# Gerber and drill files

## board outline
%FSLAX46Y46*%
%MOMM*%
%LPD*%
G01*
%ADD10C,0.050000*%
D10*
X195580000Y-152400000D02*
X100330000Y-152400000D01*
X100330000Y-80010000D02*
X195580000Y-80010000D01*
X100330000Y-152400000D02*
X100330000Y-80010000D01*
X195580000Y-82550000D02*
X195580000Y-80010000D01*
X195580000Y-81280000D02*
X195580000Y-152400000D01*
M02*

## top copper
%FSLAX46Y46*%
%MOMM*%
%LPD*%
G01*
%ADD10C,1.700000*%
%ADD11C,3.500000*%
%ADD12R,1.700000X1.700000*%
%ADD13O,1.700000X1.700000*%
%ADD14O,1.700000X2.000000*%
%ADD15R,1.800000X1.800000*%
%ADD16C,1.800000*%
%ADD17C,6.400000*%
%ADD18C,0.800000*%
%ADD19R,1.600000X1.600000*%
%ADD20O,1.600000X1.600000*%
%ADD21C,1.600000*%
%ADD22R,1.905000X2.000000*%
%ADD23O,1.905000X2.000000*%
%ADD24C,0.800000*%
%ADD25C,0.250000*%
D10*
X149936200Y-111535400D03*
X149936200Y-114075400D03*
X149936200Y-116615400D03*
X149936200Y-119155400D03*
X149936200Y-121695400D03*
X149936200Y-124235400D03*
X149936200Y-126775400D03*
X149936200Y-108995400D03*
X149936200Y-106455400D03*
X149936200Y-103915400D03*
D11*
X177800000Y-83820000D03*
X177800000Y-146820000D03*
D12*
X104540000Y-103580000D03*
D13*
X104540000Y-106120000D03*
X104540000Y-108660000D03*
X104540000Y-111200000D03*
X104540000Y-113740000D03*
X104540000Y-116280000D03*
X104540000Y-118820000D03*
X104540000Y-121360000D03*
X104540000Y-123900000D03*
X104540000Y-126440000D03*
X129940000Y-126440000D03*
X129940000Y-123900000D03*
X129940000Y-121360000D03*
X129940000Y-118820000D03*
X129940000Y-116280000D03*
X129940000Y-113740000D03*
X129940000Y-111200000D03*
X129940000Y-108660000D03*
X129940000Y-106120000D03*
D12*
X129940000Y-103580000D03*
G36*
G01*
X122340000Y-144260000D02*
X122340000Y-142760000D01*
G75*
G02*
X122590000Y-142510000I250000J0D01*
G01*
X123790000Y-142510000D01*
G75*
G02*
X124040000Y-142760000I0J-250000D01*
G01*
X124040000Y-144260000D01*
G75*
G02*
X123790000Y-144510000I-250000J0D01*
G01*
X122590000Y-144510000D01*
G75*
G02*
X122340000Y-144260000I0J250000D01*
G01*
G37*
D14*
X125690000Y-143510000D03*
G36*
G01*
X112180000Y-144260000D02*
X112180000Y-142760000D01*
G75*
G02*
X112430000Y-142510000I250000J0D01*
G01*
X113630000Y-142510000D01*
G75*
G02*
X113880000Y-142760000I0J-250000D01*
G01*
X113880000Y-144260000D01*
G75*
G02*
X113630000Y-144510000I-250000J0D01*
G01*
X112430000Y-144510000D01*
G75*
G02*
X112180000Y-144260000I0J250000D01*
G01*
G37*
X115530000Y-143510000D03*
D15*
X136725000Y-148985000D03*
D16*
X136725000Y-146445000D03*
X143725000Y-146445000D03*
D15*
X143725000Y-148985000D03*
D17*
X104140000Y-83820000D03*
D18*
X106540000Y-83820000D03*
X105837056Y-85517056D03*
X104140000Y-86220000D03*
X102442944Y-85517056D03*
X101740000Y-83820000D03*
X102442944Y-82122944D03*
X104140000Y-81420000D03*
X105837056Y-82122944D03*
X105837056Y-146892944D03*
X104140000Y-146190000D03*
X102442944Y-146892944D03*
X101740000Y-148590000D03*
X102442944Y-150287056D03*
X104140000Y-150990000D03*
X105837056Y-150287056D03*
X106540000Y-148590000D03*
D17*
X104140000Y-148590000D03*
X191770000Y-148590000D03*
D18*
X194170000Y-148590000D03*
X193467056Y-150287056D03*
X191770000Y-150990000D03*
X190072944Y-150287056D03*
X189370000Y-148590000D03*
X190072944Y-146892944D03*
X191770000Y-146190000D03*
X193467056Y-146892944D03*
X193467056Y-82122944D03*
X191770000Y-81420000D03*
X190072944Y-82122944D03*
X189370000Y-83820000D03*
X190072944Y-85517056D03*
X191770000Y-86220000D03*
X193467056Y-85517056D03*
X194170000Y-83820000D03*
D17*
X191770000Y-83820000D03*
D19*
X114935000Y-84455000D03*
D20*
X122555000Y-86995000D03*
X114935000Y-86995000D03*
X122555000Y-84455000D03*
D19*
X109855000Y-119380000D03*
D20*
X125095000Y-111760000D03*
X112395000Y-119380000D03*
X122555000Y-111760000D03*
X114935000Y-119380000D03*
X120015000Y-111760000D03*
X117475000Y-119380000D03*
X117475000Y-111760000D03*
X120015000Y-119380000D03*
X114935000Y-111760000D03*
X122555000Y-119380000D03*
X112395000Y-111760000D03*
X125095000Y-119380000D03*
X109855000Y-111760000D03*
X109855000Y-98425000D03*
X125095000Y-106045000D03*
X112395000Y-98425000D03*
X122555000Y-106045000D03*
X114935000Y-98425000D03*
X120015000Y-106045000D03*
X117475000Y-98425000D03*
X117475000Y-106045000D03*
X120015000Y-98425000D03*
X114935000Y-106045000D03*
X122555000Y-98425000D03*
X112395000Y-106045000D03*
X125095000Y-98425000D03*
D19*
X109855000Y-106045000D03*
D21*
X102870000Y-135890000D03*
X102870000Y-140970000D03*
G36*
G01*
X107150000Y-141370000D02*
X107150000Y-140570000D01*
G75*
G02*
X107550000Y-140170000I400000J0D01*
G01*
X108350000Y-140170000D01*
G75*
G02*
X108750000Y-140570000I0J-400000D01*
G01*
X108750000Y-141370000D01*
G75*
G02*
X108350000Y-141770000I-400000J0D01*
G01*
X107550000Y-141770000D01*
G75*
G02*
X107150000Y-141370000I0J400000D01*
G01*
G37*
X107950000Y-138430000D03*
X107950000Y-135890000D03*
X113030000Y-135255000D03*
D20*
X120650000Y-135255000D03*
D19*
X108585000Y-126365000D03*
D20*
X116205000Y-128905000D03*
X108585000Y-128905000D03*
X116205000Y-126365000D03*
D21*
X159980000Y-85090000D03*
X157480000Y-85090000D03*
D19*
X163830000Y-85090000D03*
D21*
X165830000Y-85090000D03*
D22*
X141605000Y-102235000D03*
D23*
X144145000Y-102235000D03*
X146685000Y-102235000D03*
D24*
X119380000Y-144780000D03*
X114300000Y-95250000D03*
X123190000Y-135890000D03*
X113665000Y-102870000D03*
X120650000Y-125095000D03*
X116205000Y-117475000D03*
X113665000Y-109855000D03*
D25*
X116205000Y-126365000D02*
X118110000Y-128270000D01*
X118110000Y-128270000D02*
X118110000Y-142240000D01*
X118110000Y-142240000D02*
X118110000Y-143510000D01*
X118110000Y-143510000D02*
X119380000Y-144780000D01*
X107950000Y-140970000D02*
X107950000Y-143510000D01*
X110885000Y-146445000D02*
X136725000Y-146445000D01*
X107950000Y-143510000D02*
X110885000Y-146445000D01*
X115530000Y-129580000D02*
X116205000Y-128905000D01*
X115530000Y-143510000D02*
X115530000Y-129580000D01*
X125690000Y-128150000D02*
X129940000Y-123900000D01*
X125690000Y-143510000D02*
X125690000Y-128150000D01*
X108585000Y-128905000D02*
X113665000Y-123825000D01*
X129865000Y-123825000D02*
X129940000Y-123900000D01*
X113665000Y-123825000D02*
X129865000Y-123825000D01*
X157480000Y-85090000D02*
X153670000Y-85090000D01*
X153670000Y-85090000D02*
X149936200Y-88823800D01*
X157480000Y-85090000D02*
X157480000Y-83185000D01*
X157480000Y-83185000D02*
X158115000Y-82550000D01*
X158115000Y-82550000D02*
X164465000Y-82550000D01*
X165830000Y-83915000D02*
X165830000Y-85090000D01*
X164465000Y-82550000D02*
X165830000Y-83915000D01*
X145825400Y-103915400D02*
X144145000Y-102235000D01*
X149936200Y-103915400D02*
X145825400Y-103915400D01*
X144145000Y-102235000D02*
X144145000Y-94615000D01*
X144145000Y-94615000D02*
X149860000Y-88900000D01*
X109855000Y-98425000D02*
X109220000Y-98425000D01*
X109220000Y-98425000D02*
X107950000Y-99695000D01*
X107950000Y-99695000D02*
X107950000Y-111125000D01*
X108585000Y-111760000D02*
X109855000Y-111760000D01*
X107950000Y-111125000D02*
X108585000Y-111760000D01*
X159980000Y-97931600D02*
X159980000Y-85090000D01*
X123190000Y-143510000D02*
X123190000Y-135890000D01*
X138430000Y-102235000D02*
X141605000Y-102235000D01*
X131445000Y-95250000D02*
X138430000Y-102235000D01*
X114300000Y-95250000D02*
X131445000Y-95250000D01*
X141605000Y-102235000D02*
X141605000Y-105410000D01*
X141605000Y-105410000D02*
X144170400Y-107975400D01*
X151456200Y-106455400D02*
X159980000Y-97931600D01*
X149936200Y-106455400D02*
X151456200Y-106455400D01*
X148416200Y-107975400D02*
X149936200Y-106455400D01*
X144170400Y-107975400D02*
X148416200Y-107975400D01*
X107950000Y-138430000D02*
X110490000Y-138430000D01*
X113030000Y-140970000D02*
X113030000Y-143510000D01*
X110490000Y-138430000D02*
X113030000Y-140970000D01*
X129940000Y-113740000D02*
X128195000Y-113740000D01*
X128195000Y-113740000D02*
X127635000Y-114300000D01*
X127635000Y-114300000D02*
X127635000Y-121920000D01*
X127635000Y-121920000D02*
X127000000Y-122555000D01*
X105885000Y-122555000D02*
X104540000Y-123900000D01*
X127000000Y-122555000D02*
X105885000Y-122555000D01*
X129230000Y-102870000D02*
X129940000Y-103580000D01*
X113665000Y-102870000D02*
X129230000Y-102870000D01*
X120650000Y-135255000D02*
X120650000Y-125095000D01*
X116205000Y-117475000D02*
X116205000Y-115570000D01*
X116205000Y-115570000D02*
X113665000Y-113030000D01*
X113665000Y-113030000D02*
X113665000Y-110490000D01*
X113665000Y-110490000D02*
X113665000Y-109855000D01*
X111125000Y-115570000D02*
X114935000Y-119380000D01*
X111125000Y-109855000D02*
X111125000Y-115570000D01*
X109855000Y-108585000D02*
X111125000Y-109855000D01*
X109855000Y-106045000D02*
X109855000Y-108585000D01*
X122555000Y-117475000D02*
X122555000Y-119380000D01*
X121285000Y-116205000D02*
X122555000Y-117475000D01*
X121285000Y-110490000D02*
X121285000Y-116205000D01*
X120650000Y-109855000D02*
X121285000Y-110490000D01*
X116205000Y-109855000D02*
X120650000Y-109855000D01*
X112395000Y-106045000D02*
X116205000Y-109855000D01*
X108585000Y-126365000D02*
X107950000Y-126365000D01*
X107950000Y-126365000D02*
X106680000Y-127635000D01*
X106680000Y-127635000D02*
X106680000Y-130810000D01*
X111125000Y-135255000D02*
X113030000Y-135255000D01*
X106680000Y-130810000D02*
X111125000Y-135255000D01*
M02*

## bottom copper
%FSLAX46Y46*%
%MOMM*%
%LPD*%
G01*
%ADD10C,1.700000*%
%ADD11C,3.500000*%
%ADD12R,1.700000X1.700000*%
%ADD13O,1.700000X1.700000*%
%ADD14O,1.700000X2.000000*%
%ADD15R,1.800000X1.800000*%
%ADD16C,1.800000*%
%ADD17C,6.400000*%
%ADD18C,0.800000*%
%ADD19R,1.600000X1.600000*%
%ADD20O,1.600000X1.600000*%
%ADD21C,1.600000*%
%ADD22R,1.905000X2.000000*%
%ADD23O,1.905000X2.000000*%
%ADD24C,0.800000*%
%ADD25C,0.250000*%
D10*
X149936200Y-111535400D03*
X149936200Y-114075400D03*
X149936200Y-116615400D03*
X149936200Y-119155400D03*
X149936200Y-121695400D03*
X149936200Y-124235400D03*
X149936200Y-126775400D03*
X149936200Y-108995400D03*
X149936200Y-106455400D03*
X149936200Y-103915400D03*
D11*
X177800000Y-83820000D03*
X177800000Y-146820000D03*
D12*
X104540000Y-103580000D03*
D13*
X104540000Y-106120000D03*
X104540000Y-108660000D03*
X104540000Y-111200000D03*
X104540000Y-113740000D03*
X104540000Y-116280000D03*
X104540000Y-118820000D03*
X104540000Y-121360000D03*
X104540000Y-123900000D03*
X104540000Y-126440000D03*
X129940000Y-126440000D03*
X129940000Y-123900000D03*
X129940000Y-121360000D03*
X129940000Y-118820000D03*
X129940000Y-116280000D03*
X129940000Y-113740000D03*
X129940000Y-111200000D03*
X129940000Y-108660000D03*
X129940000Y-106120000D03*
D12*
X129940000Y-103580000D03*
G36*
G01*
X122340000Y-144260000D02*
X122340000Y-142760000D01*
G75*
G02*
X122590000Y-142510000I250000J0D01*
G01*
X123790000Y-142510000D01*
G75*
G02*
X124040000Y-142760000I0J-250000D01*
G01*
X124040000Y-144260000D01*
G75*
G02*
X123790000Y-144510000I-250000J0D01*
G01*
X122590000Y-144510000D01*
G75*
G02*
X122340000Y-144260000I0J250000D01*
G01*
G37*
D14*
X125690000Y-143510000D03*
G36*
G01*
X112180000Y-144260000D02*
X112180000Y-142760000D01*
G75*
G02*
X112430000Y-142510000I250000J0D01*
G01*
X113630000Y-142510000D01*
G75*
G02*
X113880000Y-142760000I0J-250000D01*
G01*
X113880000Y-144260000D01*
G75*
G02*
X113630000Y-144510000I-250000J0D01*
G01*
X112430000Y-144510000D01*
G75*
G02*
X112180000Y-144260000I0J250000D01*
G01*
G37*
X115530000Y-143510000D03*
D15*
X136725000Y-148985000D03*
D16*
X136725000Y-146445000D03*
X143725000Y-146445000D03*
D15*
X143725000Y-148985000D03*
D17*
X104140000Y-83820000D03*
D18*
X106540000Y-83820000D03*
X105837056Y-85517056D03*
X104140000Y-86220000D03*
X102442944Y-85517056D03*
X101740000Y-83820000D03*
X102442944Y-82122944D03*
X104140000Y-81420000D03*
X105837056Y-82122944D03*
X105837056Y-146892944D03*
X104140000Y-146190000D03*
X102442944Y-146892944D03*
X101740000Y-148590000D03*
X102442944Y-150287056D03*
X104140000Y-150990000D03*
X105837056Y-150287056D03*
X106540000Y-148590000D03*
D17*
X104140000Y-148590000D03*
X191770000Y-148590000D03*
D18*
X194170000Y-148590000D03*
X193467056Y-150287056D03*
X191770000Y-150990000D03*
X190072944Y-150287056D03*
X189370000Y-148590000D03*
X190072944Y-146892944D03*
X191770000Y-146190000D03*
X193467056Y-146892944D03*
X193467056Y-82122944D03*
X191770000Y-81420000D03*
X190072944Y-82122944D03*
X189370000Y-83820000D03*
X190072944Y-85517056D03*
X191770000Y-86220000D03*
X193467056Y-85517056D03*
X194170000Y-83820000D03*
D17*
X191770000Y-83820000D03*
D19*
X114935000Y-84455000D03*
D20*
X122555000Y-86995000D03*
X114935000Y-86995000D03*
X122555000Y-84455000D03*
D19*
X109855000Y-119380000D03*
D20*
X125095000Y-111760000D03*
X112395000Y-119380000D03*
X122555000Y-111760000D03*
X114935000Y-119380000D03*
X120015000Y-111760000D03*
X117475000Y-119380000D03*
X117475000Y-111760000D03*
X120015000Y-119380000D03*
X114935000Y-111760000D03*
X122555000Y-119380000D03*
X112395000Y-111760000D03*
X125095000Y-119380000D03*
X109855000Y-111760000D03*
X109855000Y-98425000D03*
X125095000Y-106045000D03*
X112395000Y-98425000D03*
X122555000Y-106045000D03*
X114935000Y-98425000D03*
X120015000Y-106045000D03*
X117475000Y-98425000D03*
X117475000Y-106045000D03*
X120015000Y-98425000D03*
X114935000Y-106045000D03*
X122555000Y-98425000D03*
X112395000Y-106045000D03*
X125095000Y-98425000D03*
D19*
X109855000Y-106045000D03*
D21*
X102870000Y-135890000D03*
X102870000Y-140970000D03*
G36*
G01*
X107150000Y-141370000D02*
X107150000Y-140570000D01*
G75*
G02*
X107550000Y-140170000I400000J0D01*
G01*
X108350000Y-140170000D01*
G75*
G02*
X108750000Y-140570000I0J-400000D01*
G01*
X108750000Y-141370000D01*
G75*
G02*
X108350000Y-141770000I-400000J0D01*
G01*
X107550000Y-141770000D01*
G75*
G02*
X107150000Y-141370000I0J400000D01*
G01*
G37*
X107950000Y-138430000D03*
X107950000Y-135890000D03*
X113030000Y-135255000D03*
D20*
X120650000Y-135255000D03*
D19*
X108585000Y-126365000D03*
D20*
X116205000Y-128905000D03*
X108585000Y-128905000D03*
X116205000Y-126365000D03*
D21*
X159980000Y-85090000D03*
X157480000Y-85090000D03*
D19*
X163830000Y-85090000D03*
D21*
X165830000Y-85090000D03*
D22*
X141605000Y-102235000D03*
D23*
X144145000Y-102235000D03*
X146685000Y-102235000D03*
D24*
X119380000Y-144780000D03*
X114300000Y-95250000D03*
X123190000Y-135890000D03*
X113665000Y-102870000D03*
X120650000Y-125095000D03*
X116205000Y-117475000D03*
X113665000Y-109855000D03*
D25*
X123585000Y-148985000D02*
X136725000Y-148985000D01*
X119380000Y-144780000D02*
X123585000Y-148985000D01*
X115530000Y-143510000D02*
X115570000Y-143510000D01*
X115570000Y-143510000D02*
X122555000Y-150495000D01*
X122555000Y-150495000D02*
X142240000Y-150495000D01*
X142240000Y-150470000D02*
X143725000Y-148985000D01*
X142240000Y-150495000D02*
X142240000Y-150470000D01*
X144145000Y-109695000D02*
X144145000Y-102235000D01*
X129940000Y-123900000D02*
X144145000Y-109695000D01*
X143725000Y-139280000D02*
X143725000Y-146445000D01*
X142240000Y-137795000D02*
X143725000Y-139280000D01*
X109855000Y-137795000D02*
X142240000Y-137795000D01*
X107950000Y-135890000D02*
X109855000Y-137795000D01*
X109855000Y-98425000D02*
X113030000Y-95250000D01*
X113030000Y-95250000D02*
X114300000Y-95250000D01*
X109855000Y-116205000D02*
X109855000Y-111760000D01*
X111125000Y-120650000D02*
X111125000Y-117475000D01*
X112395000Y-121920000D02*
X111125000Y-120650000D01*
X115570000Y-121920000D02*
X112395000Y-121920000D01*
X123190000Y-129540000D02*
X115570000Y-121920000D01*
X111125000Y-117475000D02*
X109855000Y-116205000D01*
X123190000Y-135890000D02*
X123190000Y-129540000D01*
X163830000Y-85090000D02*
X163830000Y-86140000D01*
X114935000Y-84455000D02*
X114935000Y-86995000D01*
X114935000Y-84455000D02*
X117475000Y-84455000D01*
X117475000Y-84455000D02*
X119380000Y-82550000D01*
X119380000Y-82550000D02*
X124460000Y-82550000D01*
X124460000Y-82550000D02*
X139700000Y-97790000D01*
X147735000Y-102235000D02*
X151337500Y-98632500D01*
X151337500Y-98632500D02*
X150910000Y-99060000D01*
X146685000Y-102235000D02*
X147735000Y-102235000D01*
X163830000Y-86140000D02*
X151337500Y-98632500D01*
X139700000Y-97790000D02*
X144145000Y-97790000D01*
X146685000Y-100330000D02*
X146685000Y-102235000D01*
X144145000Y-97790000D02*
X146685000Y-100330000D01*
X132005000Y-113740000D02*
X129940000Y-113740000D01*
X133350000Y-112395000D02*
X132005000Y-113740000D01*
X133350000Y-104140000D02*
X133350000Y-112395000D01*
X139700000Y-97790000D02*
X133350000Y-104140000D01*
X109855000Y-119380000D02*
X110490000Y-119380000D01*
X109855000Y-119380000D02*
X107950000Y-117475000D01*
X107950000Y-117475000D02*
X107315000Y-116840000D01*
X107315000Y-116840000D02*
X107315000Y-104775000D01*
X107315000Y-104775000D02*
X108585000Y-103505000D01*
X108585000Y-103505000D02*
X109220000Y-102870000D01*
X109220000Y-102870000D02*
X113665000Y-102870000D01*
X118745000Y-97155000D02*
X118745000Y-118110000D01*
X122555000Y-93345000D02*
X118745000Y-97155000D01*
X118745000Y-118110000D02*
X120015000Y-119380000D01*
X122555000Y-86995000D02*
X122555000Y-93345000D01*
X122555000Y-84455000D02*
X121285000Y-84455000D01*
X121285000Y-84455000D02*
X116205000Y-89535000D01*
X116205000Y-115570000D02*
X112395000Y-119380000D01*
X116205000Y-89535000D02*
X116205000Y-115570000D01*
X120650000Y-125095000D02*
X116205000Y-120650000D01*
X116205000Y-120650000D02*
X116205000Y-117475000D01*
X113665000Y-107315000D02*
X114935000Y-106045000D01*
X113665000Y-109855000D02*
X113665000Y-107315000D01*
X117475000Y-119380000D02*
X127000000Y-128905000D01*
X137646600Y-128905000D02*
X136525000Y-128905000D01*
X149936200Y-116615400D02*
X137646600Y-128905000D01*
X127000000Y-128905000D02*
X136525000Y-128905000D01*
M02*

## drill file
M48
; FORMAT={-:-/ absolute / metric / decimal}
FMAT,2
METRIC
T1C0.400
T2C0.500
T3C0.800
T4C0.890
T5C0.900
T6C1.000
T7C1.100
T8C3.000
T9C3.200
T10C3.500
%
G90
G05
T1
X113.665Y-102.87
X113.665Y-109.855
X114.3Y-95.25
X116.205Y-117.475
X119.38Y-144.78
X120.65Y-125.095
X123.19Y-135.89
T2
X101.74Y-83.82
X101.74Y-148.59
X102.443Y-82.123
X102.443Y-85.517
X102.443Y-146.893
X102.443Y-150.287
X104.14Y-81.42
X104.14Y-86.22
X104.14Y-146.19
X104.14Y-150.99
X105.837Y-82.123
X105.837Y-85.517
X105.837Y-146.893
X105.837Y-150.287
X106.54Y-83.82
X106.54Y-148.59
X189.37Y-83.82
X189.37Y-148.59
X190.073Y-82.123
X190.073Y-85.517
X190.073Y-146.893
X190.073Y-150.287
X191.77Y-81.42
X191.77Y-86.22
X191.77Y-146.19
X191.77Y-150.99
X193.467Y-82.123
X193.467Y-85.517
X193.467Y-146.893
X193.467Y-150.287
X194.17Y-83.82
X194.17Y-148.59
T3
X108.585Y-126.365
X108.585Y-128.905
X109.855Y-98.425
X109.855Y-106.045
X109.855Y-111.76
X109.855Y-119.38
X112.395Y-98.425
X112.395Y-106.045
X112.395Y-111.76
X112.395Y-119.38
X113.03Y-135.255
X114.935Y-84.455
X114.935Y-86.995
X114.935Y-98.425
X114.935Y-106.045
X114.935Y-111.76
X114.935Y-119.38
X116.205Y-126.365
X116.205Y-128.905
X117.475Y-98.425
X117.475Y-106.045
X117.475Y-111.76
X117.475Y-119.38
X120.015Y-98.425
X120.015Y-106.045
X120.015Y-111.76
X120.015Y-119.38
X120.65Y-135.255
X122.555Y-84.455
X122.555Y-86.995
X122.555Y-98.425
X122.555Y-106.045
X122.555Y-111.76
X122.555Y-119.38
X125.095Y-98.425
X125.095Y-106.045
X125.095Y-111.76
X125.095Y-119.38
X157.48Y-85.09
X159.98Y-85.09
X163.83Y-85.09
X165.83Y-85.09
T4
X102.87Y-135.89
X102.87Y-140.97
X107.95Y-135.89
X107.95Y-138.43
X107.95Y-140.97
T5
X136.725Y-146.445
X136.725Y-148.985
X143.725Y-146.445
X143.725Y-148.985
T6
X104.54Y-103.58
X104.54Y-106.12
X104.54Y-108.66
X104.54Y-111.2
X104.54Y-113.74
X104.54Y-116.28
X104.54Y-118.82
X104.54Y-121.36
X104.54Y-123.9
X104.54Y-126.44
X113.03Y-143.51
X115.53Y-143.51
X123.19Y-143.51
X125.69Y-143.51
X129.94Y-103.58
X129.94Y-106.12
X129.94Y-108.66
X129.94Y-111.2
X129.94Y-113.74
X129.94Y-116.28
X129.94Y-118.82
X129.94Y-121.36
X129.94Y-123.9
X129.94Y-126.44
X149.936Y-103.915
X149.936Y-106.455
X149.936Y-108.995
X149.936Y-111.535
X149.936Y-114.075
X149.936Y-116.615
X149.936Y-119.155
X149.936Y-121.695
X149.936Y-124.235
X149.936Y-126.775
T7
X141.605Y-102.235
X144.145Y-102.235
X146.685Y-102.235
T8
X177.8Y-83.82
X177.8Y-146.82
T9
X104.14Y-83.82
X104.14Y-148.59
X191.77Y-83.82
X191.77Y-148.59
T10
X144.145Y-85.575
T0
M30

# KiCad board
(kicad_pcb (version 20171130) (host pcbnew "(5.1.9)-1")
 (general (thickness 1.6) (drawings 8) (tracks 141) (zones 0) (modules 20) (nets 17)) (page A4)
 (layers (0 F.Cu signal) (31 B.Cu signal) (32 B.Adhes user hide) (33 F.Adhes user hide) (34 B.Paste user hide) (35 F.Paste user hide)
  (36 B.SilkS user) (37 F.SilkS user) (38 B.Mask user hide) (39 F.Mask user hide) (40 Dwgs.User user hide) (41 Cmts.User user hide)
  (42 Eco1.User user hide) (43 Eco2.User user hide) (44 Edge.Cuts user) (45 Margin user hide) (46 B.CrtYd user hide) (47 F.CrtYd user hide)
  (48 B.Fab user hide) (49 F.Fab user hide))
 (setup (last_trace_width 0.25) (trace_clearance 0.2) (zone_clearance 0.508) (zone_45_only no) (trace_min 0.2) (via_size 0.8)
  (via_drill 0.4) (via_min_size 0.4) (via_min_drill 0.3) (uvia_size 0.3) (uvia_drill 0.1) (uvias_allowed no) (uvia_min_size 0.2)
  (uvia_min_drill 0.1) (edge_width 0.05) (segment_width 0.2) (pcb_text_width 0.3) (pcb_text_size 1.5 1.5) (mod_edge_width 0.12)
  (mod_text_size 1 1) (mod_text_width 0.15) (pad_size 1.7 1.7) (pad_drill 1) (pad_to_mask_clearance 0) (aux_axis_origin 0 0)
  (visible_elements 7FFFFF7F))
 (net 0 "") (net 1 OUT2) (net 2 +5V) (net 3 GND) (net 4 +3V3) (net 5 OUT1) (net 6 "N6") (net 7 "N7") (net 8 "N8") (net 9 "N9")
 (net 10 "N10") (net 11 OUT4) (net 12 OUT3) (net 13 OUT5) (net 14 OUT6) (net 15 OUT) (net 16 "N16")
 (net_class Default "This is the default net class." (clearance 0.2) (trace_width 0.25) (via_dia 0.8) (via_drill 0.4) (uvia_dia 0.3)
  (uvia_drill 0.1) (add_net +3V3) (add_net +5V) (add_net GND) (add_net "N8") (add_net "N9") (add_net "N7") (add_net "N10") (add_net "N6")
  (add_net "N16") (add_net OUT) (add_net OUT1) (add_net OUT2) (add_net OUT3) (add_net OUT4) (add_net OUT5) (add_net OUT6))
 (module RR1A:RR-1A (layer F.Cu) (at 177.8 115.32 270)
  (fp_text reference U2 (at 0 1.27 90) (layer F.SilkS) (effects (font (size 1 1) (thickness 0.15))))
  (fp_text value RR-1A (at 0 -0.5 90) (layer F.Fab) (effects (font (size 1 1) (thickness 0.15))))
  (pad 4 thru_hole circle (at -3.7846 27.8638 270) (size 1.7 1.7) (drill 1) (layers *.Cu *.Mask))
  (pad 5 thru_hole circle (at -1.2446 27.8638 270) (size 1.7 1.7) (drill 1) (layers *.Cu *.Mask))
  (pad 6 thru_hole circle (at 1.2954 27.8638 270) (size 1.7 1.7) (drill 1) (layers *.Cu *.Mask) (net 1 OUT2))
  (pad 7 thru_hole circle (at 3.8354 27.8638 270) (size 1.7 1.7) (drill 1) (layers *.Cu *.Mask))
  (pad 8 thru_hole circle (at 6.3754 27.8638 270) (size 1.7 1.7) (drill 1) (layers *.Cu *.Mask))
  (pad 9 thru_hole circle (at 8.9154 27.8638 270) (size 1.7 1.7) (drill 1) (layers *.Cu *.Mask))
  (pad 10 thru_hole circle (at 11.4554 27.8638 270) (size 1.7 1.7) (drill 1) (layers *.Cu *.Mask))
  (pad 3 thru_hole circle (at -6.3246 27.8638 270) (size 1.7 1.7) (drill 1) (layers *.Cu *.Mask))
  (pad 2 thru_hole circle (at -8.8646 27.8638 270) (size 1.7 1.7) (drill 1) (layers *.Cu *.Mask) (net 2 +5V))
  (pad 1 thru_hole circle (at -11.4046 27.8638 270) (size 1.7 1.7) (drill 1) (layers *.Cu *.Mask) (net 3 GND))
  (pad 11 thru_hole circle (at -31.5 0 270) (size 3.5 3.5) (drill 3) (layers *.Cu *.Mask))
  (pad 12 thru_hole circle (at 31.5 0 270) (size 3.5 3.5) (drill 3) (layers *.Cu *.Mask)))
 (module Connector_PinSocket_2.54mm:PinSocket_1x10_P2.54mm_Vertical (layer F.Cu) (at 104.54 103.58)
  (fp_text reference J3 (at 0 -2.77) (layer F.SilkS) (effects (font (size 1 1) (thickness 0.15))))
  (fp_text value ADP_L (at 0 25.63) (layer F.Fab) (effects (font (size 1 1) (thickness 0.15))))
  (pad 1 thru_hole rect (at 0 0) (size 1.7 1.7) (drill 1) (layers *.Cu *.Mask))
  (pad 2 thru_hole oval (at 0 2.54) (size 1.7 1.7) (drill 1) (layers *.Cu *.Mask))
  (pad 3 thru_hole oval (at 0 5.08) (size 1.7 1.7) (drill 1) (layers *.Cu *.Mask))
  (pad 4 thru_hole oval (at 0 7.62) (size 1.7 1.7) (drill 1) (layers *.Cu *.Mask))
  (pad 5 thru_hole oval (at 0 10.16) (size 1.7 1.7) (drill 1) (layers *.Cu *.Mask))
  (pad 6 thru_hole oval (at 0 12.7) (size 1.7 1.7) (drill 1) (layers *.Cu *.Mask))
  (pad 7 thru_hole oval (at 0 15.24) (size 1.7 1.7) (drill 1) (layers *.Cu *.Mask))
  (pad 8 thru_hole oval (at 0 17.78) (size 1.7 1.7) (drill 1) (layers *.Cu *.Mask))
  (pad 9 thru_hole oval (at 0 20.32) (size 1.7 1.7) (drill 1) (layers *.Cu *.Mask) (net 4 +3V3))
  (pad 10 thru_hole oval (at 0 22.86) (size 1.7 1.7) (drill 1) (layers *.Cu *.Mask)))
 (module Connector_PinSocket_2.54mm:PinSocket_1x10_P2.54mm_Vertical (layer F.Cu) (at 129.94 103.58)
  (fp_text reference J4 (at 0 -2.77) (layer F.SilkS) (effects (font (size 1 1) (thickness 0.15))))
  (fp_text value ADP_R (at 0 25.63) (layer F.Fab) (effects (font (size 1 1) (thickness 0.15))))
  (pad 10 thru_hole oval (at 0 22.86) (size 1.7 1.7) (drill 1) (layers *.Cu *.Mask))
  (pad 9 thru_hole oval (at 0 20.32) (size 1.7 1.7) (drill 1) (layers *.Cu *.Mask) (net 3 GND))
  (pad 8 thru_hole oval (at 0 17.78) (size 1.7 1.7) (drill 1) (layers *.Cu *.Mask))
  (pad 7 thru_hole oval (at 0 15.24) (size 1.7 1.7) (drill 1) (layers *.Cu *.Mask))
  (pad 6 thru_hole oval (at 0 12.7) (size 1.7 1.7) (drill 1) (layers *.Cu *.Mask))
  (pad 5 thru_hole oval (at 0 10.16) (size 1.7 1.7) (drill 1) (layers *.Cu *.Mask) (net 4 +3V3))
  (pad 4 thru_hole oval (at 0 7.62) (size 1.7 1.7) (drill 1) (layers *.Cu *.Mask))
  (pad 3 thru_hole oval (at 0 5.08) (size 1.7 1.7) (drill 1) (layers *.Cu *.Mask))
  (pad 2 thru_hole oval (at 0 2.54) (size 1.7 1.7) (drill 1) (layers *.Cu *.Mask))
  (pad 1 thru_hole rect (at 0 0) (size 1.7 1.7) (drill 1) (layers *.Cu *.Mask) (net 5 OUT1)))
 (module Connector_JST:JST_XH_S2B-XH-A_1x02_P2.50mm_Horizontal (layer F.Cu) (at 123.19 143.51)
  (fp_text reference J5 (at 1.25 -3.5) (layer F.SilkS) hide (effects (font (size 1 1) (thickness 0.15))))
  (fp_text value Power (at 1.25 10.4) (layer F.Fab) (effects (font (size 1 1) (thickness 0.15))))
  (pad 1 thru_hole roundrect (at 0 0) (size 1.7 2) (drill 1) (layers *.Cu *.Mask) (roundrect_rratio 0.1470588235294118) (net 2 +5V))
  (pad 2 thru_hole oval (at 2.5 0) (size 1.7 2) (drill 1) (layers *.Cu *.Mask) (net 3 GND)))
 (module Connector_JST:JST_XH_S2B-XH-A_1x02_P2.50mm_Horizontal (layer F.Cu) (at 113.03 143.51)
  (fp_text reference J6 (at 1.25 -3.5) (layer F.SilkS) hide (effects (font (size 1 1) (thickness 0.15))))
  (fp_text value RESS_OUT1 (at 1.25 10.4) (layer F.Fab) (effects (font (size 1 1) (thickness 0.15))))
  (pad 1 thru_hole roundrect (at 0 0) (size 1.7 2) (drill 1) (layers *.Cu *.Mask) (roundrect_rratio 0.1470588235294118) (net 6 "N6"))
  (pad 2 thru_hole oval (at 2.5 0) (size 1.7 2) (drill 1) (layers *.Cu *.Mask) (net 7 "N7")))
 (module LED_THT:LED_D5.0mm (layer F.Cu) (at 136.725 148.985 90)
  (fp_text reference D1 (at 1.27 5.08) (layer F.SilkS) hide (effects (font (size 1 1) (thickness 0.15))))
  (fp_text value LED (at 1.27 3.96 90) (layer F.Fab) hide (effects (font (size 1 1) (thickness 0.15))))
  (pad 1 thru_hole rect (at 0 0 90) (size 1.8 1.8) (drill 0.9) (layers *.Cu *.Mask) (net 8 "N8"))
  (pad 2 thru_hole circle (at 2.54 0 90) (size 1.8 1.8) (drill 0.9) (layers *.Cu *.Mask) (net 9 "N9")))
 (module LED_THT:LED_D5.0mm (layer F.Cu) (at 143.725 148.985 90)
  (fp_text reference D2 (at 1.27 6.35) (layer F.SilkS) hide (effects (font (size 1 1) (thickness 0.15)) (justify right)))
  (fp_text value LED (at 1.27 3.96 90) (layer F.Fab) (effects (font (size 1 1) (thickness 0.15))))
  (pad 2 thru_hole circle (at 2.54 0 90) (size 1.8 1.8) (drill 0.9) (layers *.Cu *.Mask) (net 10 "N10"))
  (pad 1 thru_hole rect (at 0 0 90) (size 1.8 1.8) (drill 0.9) (layers *.Cu *.Mask) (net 7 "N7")))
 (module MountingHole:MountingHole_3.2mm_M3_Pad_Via (layer F.Cu) (at 104.14 83.82)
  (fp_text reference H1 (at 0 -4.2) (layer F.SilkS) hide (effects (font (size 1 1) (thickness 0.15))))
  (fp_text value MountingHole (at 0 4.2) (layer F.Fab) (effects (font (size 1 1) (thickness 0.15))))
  (pad 1 thru_hole circle (at 0 0) (size 6.4 6.4) (drill 3.2) (layers *.Cu *.Mask))
  (pad 1 thru_hole circle (at 2.4 0) (size 0.8 0.8) (drill 0.5) (layers *.Cu *.Mask))
  (pad 1 thru_hole circle (at 1.697056 1.697056) (size 0.8 0.8) (drill 0.5) (layers *.Cu *.Mask))
  (pad 1 thru_hole circle (at 0 2.4) (size 0.8 0.8) (drill 0.5) (layers *.Cu *.Mask))
  (pad 1 thru_hole circle (at -1.697056 1.697056) (size 0.8 0.8) (drill 0.5) (layers *.Cu *.Mask))
  (pad 1 thru_hole circle (at -2.4 0) (size 0.8 0.8) (drill 0.5) (layers *.Cu *.Mask))
  (pad 1 thru_hole circle (at -1.697056 -1.697056) (size 0.8 0.8) (drill 0.5) (layers *.Cu *.Mask))
  (pad 1 thru_hole circle (at 0 -2.4) (size 0.8 0.8) (drill 0.5) (layers *.Cu *.Mask))
  (pad 1 thru_hole circle (at 1.697056 -1.697056) (size 0.8 0.8) (drill 0.5) (layers *.Cu *.Mask)))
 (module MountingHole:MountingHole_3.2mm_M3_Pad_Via (layer F.Cu) (at 104.14 148.59)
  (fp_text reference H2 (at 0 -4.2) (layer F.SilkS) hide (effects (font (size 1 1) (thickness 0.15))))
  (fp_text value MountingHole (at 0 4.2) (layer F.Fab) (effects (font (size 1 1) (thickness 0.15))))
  (pad 1 thru_hole circle (at 1.697056 -1.697056) (size 0.8 0.8) (drill 0.5) (layers *.Cu *.Mask))
  (pad 1 thru_hole circle (at 0 -2.4) (size 0.8 0.8) (drill 0.5) (layers *.Cu *.Mask))
  (pad 1 thru_hole circle (at -1.697056 -1.697056) (size 0.8 0.8) (drill 0.5) (layers *.Cu *.Mask))
  (pad 1 thru_hole circle (at -2.4 0) (size 0.8 0.8) (drill 0.5) (layers *.Cu *.Mask))
  (pad 1 thru_hole circle (at -1.697056 1.697056) (size 0.8 0.8) (drill 0.5) (layers *.Cu *.Mask))
  (pad 1 thru_hole circle (at 0 2.4) (size 0.8 0.8) (drill 0.5) (layers *.Cu *.Mask))
  (pad 1 thru_hole circle (at 1.697056 1.697056) (size 0.8 0.8) (drill 0.5) (layers *.Cu *.Mask))
  (pad 1 thru_hole circle (at 2.4 0) (size 0.8 0.8) (drill 0.5) (layers *.Cu *.Mask))
  (pad 1 thru_hole circle (at 0 0) (size 6.4 6.4) (drill 3.2) (layers *.Cu *.Mask)))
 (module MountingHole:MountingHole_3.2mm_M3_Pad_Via (layer F.Cu) (at 191.77 148.59)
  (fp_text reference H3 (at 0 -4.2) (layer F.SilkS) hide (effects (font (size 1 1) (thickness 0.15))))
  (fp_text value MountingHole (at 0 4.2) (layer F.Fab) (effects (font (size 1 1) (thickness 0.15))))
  (pad 1 thru_hole circle (at 0 0) (size 6.4 6.4) (drill 3.2) (layers *.Cu *.Mask))
  (pad 1 thru_hole circle (at 2.4 0) (size 0.8 0.8) (drill 0.5) (layers *.Cu *.Mask))
  (pad 1 thru_hole circle (at 1.697056 1.697056) (size 0.8 0.8) (drill 0.5) (layers *.Cu *.Mask))
  (pad 1 thru_hole circle (at 0 2.4) (size 0.8 0.8) (drill 0.5) (layers *.Cu *.Mask))
  (pad 1 thru_hole circle (at -1.697056 1.697056) (size 0.8 0.8) (drill 0.5) (layers *.Cu *.Mask))
  (pad 1 thru_hole circle (at -2.4 0) (size 0.8 0.8) (drill 0.5) (layers *.Cu *.Mask))
  (pad 1 thru_hole circle (at -1.697056 -1.697056) (size 0.8 0.8) (drill 0.5) (layers *.Cu *.Mask))
  (pad 1 thru_hole circle (at 0 -2.4) (size 0.8 0.8) (drill 0.5) (layers *.Cu *.Mask))
  (pad 1 thru_hole circle (at 1.697056 -1.697056) (size 0.8 0.8) (drill 0.5) (layers *.Cu *.Mask)))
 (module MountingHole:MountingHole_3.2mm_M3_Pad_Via (layer F.Cu) (at 191.77 83.82)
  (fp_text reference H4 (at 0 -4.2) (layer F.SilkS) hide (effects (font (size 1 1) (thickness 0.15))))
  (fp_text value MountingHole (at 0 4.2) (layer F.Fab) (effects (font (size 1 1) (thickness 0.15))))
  (pad 1 thru_hole circle (at 1.697056 -1.697056) (size 0.8 0.8) (drill 0.5) (layers *.Cu *.Mask))
  (pad 1 thru_hole circle (at 0 -2.4) (size 0.8 0.8) (drill 0.5) (layers *.Cu *.Mask))
  (pad 1 thru_hole circle (at -1.697056 -1.697056) (size 0.8 0.8) (drill 0.5) (layers *.Cu *.Mask))
  (pad 1 thru_hole circle (at -2.4 0) (size 0.8 0.8) (drill 0.5) (layers *.Cu *.Mask))
  (pad 1 thru_hole circle (at -1.697056 1.697056) (size 0.8 0.8) (drill 0.5) (layers *.Cu *.Mask))
  (pad 1 thru_hole circle (at 0 2.4) (size 0.8 0.8) (drill 0.5) (layers *.Cu *.Mask))
  (pad 1 thru_hole circle (at 1.697056 1.697056) (size 0.8 0.8) (drill 0.5) (layers *.Cu *.Mask))
  (pad 1 thru_hole circle (at 2.4 0) (size 0.8 0.8) (drill 0.5) (layers *.Cu *.Mask))
  (pad 1 thru_hole circle (at 0 0) (size 6.4 6.4) (drill 3.2) (layers *.Cu *.Mask)))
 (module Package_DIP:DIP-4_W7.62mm (layer F.Cu) (at 114.935 84.455)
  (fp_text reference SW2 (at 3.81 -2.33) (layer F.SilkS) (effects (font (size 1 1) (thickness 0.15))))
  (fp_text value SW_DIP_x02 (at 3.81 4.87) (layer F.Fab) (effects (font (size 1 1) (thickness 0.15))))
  (pad 1 thru_hole rect (at 0 0) (size 1.6 1.6) (drill 0.8) (layers *.Cu *.Mask) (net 4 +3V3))
  (pad 3 thru_hole oval (at 7.62 2.54) (size 1.6 1.6) (drill 0.8) (layers *.Cu *.Mask) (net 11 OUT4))
  (pad 2 thru_hole oval (at 0 2.54) (size 1.6 1.6) (drill 0.8) (layers *.Cu *.Mask) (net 4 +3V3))
  (pad 4 thru_hole oval (at 7.62 0) (size 1.6 1.6) (drill 0.8) (layers *.Cu *.Mask) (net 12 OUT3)))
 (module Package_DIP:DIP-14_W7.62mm (layer F.Cu) (at 109.855 119.38 90)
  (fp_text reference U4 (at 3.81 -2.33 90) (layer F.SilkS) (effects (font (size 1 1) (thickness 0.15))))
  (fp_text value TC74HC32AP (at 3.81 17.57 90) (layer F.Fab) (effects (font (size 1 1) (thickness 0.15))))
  (pad 1 thru_hole rect (at 0 0 90) (size 1.6 1.6) (drill 0.8) (layers *.Cu *.Mask) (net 5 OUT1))
  (pad 8 thru_hole oval (at 7.62 15.24 90) (size 1.6 1.6) (drill 0.8) (layers *.Cu *.Mask))
  (pad 2 thru_hole oval (at 0 2.54 90) (size 1.6 1.6) (drill 0.8) (layers *.Cu *.Mask) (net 12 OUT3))
  (pad 9 thru_hole oval (at 7.62 12.7 90) (size 1.6 1.6) (drill 0.8) (layers *.Cu *.Mask))
  (pad 3 thru_hole oval (at 0 5.08 90) (size 1.6 1.6) (drill 0.8) (layers *.Cu *.Mask) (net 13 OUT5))
  (pad 10 thru_hole oval (at 7.62 10.16 90) (size 1.6 1.6) (drill 0.8) (layers *.Cu *.Mask))
  (pad 4 thru_hole oval (at 0 7.62 90) (size 1.6 1.6) (drill 0.8) (layers *.Cu *.Mask) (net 1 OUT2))
  (pad 11 thru_hole oval (at 7.62 7.62 90) (size 1.6 1.6) (drill 0.8) (layers *.Cu *.Mask))
  (pad 5 thru_hole oval (at 0 10.16 90) (size 1.6 1.6) (drill 0.8) (layers *.Cu *.Mask) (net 11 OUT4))
  (pad 12 thru_hole oval (at 7.62 5.08 90) (size 1.6 1.6) (drill 0.8) (layers *.Cu *.Mask))
  (pad 6 thru_hole oval (at 0 12.7 90) (size 1.6 1.6) (drill 0.8) (layers *.Cu *.Mask) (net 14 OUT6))
  (pad 13 thru_hole oval (at 7.62 2.54 90) (size 1.6 1.6) (drill 0.8) (layers *.Cu *.Mask))
  (pad 7 thru_hole oval (at 0 15.24 90) (size 1.6 1.6) (drill 0.8) (layers *.Cu *.Mask))
  (pad 14 thru_hole oval (at 7.62 0 90) (size 1.6 1.6) (drill 0.8) (layers *.Cu *.Mask) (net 2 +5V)))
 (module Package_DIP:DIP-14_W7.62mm (layer F.Cu) (at 109.855 106.045 90)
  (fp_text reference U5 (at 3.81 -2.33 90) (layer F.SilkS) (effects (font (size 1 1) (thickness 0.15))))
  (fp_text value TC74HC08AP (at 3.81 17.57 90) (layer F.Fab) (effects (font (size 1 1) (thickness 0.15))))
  (pad 14 thru_hole oval (at 7.62 0 90) (size 1.6 1.6) (drill 0.8) (layers *.Cu *.Mask) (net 2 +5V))
  (pad 7 thru_hole oval (at 0 15.24 90) (size 1.6 1.6) (drill 0.8) (layers *.Cu *.Mask))
  (pad 13 thru_hole oval (at 7.62 2.54 90) (size 1.6 1.6) (drill 0.8) (layers *.Cu *.Mask))
  (pad 6 thru_hole oval (at 0 12.7 90) (size 1.6 1.6) (drill 0.8) (layers *.Cu *.Mask))
  (pad 12 thru_hole oval (at 7.62 5.08 90) (size 1.6 1.6) (drill 0.8) (layers *.Cu *.Mask))
  (pad 5 thru_hole oval (at 0 10.16 90) (size 1.6 1.6) (drill 0.8) (layers *.Cu *.Mask))
  (pad 11 thru_hole oval (at 7.62 7.62 90) (size 1.6 1.6) (drill 0.8) (layers *.Cu *.Mask))
  (pad 4 thru_hole oval (at 0 7.62 90) (size 1.6 1.6) (drill 0.8) (layers *.Cu *.Mask))
  (pad 10 thru_hole oval (at 7.62 10.16 90) (size 1.6 1.6) (drill 0.8) (layers *.Cu *.Mask))
  (pad 3 thru_hole oval (at 0 5.08 90) (size 1.6 1.6) (drill 0.8) (layers *.Cu *.Mask) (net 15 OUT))
  (pad 9 thru_hole oval (at 7.62 12.7 90) (size 1.6 1.6) (drill 0.8) (layers *.Cu *.Mask))
  (pad 2 thru_hole oval (at 0 2.54 90) (size 1.6 1.6) (drill 0.8) (layers *.Cu *.Mask) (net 14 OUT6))
  (pad 8 thru_hole oval (at 7.62 15.24 90) (size 1.6 1.6) (drill 0.8) (layers *.Cu *.Mask))
  (pad 1 thru_hole rect (at 0 0 90) (size 1.6 1.6) (drill 0.8) (layers *.Cu *.Mask) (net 13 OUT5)))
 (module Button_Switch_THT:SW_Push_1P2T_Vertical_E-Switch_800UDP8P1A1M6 (layer F.Cu) (at 107.95 140.97 180)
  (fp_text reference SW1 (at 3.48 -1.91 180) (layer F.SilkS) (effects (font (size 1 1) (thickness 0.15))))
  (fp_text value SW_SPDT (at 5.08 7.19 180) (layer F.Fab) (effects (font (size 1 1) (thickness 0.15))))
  (pad "" thru_hole circle (at 5.08 5.08) (size 1.6 1.6) (drill 0.89) (layers *.Cu *.Mask))
  (pad "" thru_hole circle (at 5.08 0) (size 1.6 1.6) (drill 0.89) (layers *.Cu *.Mask))
  (pad 1 thru_hole roundrect (at 0 0) (size 1.6 1.6) (drill 0.89) (layers *.Cu *.Mask) (roundrect_rratio 0.25) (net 9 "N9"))
  (pad 2 thru_hole circle (at 0 2.54) (size 1.6 1.6) (drill 0.89) (layers *.Cu *.Mask) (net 6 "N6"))
  (pad 3 thru_hole circle (at 0 5.08) (size 1.6 1.6) (drill 0.89) (layers *.Cu *.Mask) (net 10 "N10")))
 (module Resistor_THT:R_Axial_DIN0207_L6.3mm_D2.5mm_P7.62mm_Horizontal (layer F.Cu) (at 113.03 135.255)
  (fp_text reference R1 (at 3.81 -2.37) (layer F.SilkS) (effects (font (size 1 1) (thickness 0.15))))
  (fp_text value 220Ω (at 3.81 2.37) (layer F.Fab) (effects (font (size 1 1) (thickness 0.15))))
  (pad 1 thru_hole circle (at 0 0) (size 1.6 1.6) (drill 0.8) (layers *.Cu *.Mask) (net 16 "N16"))
  (pad 2 thru_hole oval (at 7.62 0) (size 1.6 1.6) (drill 0.8) (layers *.Cu *.Mask) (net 15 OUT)))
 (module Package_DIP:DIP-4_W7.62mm (layer F.Cu) (at 108.585 126.365)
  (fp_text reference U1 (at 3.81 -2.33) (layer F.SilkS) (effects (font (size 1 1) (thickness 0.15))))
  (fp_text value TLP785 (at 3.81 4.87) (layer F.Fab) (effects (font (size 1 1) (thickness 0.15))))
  (pad 1 thru_hole rect (at 0 0) (size 1.6 1.6) (drill 0.8) (layers *.Cu *.Mask) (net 16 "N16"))
  (pad 3 thru_hole oval (at 7.62 2.54) (size 1.6 1.6) (drill 0.8) (layers *.Cu *.Mask) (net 7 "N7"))
  (pad 2 thru_hole oval (at 0 2.54) (size 1.6 1.6) (drill 0.8) (layers *.Cu *.Mask) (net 3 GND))
  (pad 4 thru_hole oval (at 7.62 0) (size 1.6 1.6) (drill 0.8) (layers *.Cu *.Mask) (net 8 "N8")))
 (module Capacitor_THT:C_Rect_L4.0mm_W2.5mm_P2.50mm (layer F.Cu) (at 159.98 85.09 180)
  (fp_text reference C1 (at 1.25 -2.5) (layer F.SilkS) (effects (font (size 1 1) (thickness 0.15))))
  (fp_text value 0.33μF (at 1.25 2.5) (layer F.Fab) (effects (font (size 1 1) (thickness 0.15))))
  (pad 1 thru_hole circle (at 0 0 180) (size 1.6 1.6) (drill 0.8) (layers *.Cu *.Mask) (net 2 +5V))
  (pad 2 thru_hole circle (at 2.5 0 180) (size 1.6 1.6) (drill 0.8) (layers *.Cu *.Mask) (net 3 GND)))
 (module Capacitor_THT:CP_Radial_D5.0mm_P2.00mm (layer F.Cu) (at 163.83 85.09)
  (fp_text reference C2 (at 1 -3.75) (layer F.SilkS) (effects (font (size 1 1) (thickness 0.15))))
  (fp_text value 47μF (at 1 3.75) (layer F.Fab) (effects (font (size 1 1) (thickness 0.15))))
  (pad 1 thru_hole rect (at 0 0) (size 1.6 1.6) (drill 0.8) (layers *.Cu *.Mask) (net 4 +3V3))
  (pad 2 thru_hole circle (at 2 0) (size 1.6 1.6) (drill 0.8) (layers *.Cu *.Mask) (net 3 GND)))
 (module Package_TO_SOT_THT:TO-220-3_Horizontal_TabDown (layer F.Cu) (at 141.605 102.235)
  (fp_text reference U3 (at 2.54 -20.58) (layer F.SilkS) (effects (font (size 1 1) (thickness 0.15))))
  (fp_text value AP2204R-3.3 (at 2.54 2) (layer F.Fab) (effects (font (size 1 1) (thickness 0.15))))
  (pad "" np_thru_hole oval (at 2.54 -16.66) (size 3.5 3.5) (drill 3.5) (layers *.Cu *.Mask))
  (pad 1 thru_hole rect (at 0 0) (size 1.905 2) (drill 1.1) (layers *.Cu *.Mask) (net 2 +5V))
  (pad 2 thru_hole oval (at 2.54 0) (size 1.905 2) (drill 1.1) (layers *.Cu *.Mask) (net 3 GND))
  (pad 3 thru_hole oval (at 5.08 0) (size 1.905 2) (drill 1.1) (layers *.Cu *.Mask) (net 4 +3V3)))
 (gr_line (start 195.58 152.4) (end 100.33 152.4) (layer Edge.Cuts) (width 0.05))
 (gr_line (start 100.33 80.01) (end 195.58 80.01) (layer Edge.Cuts) (width 0.05))
 (gr_line (start 100.33 152.4) (end 100.33 80.01) (layer Edge.Cuts) (width 0.05))
 (gr_line (start 195.58 82.55) (end 195.58 80.01) (layer Edge.Cuts) (width 0.05))
 (gr_line (start 195.58 81.28) (end 195.58 152.4) (layer Edge.Cuts) (width 0.05))
 (segment (start 116.205 126.365) (end 118.11 128.27) (width 0.25) (layer F.Cu) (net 8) (status 10))
 (segment (start 118.11 128.27) (end 118.11 142.24) (width 0.25) (layer F.Cu) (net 8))
 (segment (start 118.11 142.24) (end 118.11 143.51) (width 0.25) (layer F.Cu) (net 8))
 (segment (start 118.11 143.51) (end 119.38 144.78) (width 0.25) (layer F.Cu) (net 8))
 (via (at 119.38 144.78) (size 0.8) (drill 0.4) (layers F.Cu B.Cu) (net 8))
 (segment (start 123.585 148.985) (end 136.725 148.985) (width 0.25) (layer B.Cu) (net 8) (status 20))
 (segment (start 119.38 144.78) (end 123.585 148.985) (width 0.25) (layer B.Cu) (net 8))
 (segment (start 107.95 140.97) (end 107.95 143.51) (width 0.25) (layer F.Cu) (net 9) (status 10))
 (segment (start 110.885 146.445) (end 136.725 146.445) (width 0.25) (layer F.Cu) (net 9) (status 20))
 (segment (start 107.95 143.51) (end 110.885 146.445) (width 0.25) (layer F.Cu) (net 9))
 (segment (start 115.53 143.51) (end 115.57 143.51) (width 0.25) (layer B.Cu) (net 7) (status 30))
 (segment (start 115.57 143.51) (end 122.555 150.495) (width 0.25) (layer B.Cu) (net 7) (status 10))
 (segment (start 122.555 150.495) (end 142.24 150.495) (width 0.25) (layer B.Cu) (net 7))
 (segment (start 142.24 150.47) (end 143.725 148.985) (width 0.25) (layer B.Cu) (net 7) (status 20))
 (segment (start 142.24 150.495) (end 142.24 150.47) (width 0.25) (layer B.Cu) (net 7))
 (segment (start 115.53 129.58) (end 116.205 128.905) (width 0.25) (layer F.Cu) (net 7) (status 20))
 (segment (start 115.53 143.51) (end 115.53 129.58) (width 0.25) (layer F.Cu) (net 7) (status 10))
 (segment (start 125.69 128.15) (end 129.94 123.9) (width 0.25) (layer F.Cu) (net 3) (status 20))
 (segment (start 125.69 143.51) (end 125.69 128.15) (width 0.25) (layer F.Cu) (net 3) (status 10))
 (segment (start 108.585 128.905) (end 113.665 123.825) (width 0.25) (layer F.Cu) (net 3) (status 10))
 (segment (start 129.865 123.825) (end 129.94 123.9) (width 0.25) (layer F.Cu) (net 3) (status 30))
 (segment (start 113.665 123.825) (end 129.865 123.825) (width 0.25) (layer F.Cu) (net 3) (status 20))
 (segment (start 157.48 85.09) (end 153.67 85.09) (width 0.25) (layer F.Cu) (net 3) (status 10))
 (segment (start 153.67 85.09) (end 149.9362 88.8238) (width 0.25) (layer F.Cu) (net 3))
 (segment (start 157.48 85.09) (end 157.48 83.185) (width 0.25) (layer F.Cu) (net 3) (status 10))
 (segment (start 157.48 83.185) (end 158.115 82.55) (width 0.25) (layer F.Cu) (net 3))
 (segment (start 158.115 82.55) (end 164.465 82.55) (width 0.25) (layer F.Cu) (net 3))
 (segment (start 165.83 83.915) (end 165.83 85.09) (width 0.25) (layer F.Cu) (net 3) (status 20))
 (segment (start 164.465 82.55) (end 165.83 83.915) (width 0.25) (layer F.Cu) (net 3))
 (segment (start 144.145 109.695) (end 144.145 102.235) (width 0.25) (layer B.Cu) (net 3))
 (segment (start 129.94 123.9) (end 144.145 109.695) (width 0.25) (layer B.Cu) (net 3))
 (segment (start 145.8254 103.9154) (end 144.145 102.235) (width 0.25) (layer F.Cu) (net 3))
 (segment (start 149.9362 103.9154) (end 145.8254 103.9154) (width 0.25) (layer F.Cu) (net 3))
 (segment (start 144.145 102.235) (end 144.145 94.615) (width 0.25) (layer F.Cu) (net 3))
 (segment (start 144.145 94.615) (end 149.86 88.9) (width 0.25) (layer F.Cu) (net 3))
 (segment (start 143.725 139.28) (end 143.725 146.445) (width 0.25) (layer B.Cu) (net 10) (status 20))
 (segment (start 142.24 137.795) (end 143.725 139.28) (width 0.25) (layer B.Cu) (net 10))
 (segment (start 109.855 137.795) (end 142.24 137.795) (width 0.25) (layer B.Cu) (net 10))
 (segment (start 107.95 135.89) (end 109.855 137.795) (width 0.25) (layer B.Cu) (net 10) (status 10))
 (segment (start 109.855 98.425) (end 109.22 98.425) (width 0.25) (layer F.Cu) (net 2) (status 30))
 (segment (start 109.22 98.425) (end 107.95 99.695) (width 0.25) (layer F.Cu) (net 2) (status 10))
 (segment (start 107.95 99.695) (end 107.95 111.125) (width 0.25) (layer F.Cu) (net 2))
 (segment (start 108.585 111.76) (end 109.855 111.76) (width 0.25) (layer F.Cu) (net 2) (status 20))
 (segment (start 107.95 111.125) (end 108.585 111.76) (width 0.25) (layer F.Cu) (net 2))
 (segment (start 159.98 97.9316) (end 159.98 85.09) (width 0.25) (layer F.Cu) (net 2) (status 20))
 (segment (start 109.855 98.425) (end 113.03 95.25) (width 0.25) (layer B.Cu) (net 2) (status 10))
 (segment (start 113.03 95.25) (end 114.3 95.25) (width 0.25) (layer B.Cu) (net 2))
 (via (at 114.3 95.25) (size 0.8) (drill 0.4) (layers F.Cu B.Cu) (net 2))
 (segment (start 123.19 143.51) (end 123.19 135.89) (width 0.25) (layer F.Cu) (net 2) (status 10))
 (via (at 123.19 135.89) (size 0.8) (drill 0.4) (layers F.Cu B.Cu) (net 2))
 (segment (start 109.855 116.205) (end 109.855 111.76) (width 0.25) (layer B.Cu) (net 2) (status 20))
 (segment (start 111.125 120.65) (end 111.125 117.475) (width 0.25) (layer B.Cu) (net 2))
 (segment (start 112.395 121.92) (end 111.125 120.65) (width 0.25) (layer B.Cu) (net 2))
 (segment (start 115.57 121.92) (end 112.395 121.92) (width 0.25) (layer B.Cu) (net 2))
 (segment (start 123.19 129.54) (end 115.57 121.92) (width 0.25) (layer B.Cu) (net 2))
 (segment (start 111.125 117.475) (end 109.855 116.205) (width 0.25) (layer B.Cu) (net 2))
 (segment (start 123.19 135.89) (end 123.19 129.54) (width 0.25) (layer B.Cu) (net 2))
 (segment (start 138.43 102.235) (end 141.605 102.235) (width 0.25) (layer F.Cu) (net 2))
 (segment (start 131.445 95.25) (end 138.43 102.235) (width 0.25) (layer F.Cu) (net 2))
 (segment (start 114.3 95.25) (end 131.445 95.25) (width 0.25) (layer F.Cu) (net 2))
 (segment (start 141.605 102.235) (end 141.605 105.41) (width 0.25) (layer F.Cu) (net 2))
 (segment (start 141.605 105.41) (end 144.1704 107.9754) (width 0.25) (layer F.Cu) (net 2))
 (segment (start 151.4562 106.4554) (end 159.98 97.9316) (width 0.25) (layer F.Cu) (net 2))
 (segment (start 149.9362 106.4554) (end 151.4562 106.4554) (width 0.25) (layer F.Cu) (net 2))
 (segment (start 148.4162 107.9754) (end 149.9362 106.4554) (width 0.25) (layer F.Cu) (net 2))
 (segment (start 144.1704 107.9754) (end 148.4162 107.9754) (width 0.25) (layer F.Cu) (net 2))
 (segment (start 107.95 138.43) (end 110.49 138.43) (width 0.25) (layer F.Cu) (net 6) (status 10))
 (segment (start 113.03 140.97) (end 113.03 143.51) (width 0.25) (layer F.Cu) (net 6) (status 20))
 (segment (start 110.49 138.43) (end 113.03 140.97) (width 0.25) (layer F.Cu) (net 6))
 (segment (start 163.83 85.09) (end 163.83 86.14) (width 0.25) (layer B.Cu) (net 4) (status 10))
 (segment (start 114.935 84.455) (end 114.935 86.995) (width 0.25) (layer B.Cu) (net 4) (status 30))
 (segment (start 114.935 84.455) (end 117.475 84.455) (width 0.25) (layer B.Cu) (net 4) (status 10))
 (segment (start 117.475 84.455) (end 119.38 82.55) (width 0.25) (layer B.Cu) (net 4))
 (segment (start 119.38 82.55) (end 124.46 82.55) (width 0.25) (layer B.Cu) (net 4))
 (segment (start 124.46 82.55) (end 139.7 97.79) (width 0.25) (layer B.Cu) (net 4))
 (segment (start 129.94 113.74) (end 128.195 113.74) (width 0.25) (layer F.Cu) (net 4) (status 10))
 (segment (start 128.195 113.74) (end 127.635 114.3) (width 0.25) (layer F.Cu) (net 4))
 (segment (start 127.635 114.3) (end 127.635 121.92) (width 0.25) (layer F.Cu) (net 4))
 (segment (start 127.635 121.92) (end 127 122.555) (width 0.25) (layer F.Cu) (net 4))
 (segment (start 105.885 122.555) (end 104.54 123.9) (width 0.25) (layer F.Cu) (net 4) (status 20))
 (segment (start 127 122.555) (end 105.885 122.555) (width 0.25) (layer F.Cu) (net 4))
 (segment (start 147.735 102.235) (end 151.3375 98.6325) (width 0.25) (layer B.Cu) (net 4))
 (segment (start 151.3375 98.6325) (end 150.91 99.06) (width 0.25) (layer B.Cu) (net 4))
 (segment (start 146.685 102.235) (end 147.735 102.235) (width 0.25) (layer B.Cu) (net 4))
 (segment (start 163.83 86.14) (end 151.3375 98.6325) (width 0.25) (layer B.Cu) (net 4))
 (segment (start 139.7 97.79) (end 144.145 97.79) (width 0.25) (layer B.Cu) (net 4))
 (segment (start 146.685 100.33) (end 146.685 102.235) (width 0.25) (layer B.Cu) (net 4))
 (segment (start 144.145 97.79) (end 146.685 100.33) (width 0.25) (layer B.Cu) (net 4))
 (segment (start 132.005 113.74) (end 129.94 113.74) (width 0.25) (layer B.Cu) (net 4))
 (segment (start 133.35 112.395) (end 132.005 113.74) (width 0.25) (layer B.Cu) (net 4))
 (segment (start 133.35 104.14) (end 133.35 112.395) (width 0.25) (layer B.Cu) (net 4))
 (segment (start 139.7 97.79) (end 133.35 104.14) (width 0.25) (layer B.Cu) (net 4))
 (segment (start 109.855 119.38) (end 110.49 119.38) (width 0.25) (layer B.Cu) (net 5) (status 30))
 (segment (start 109.855 119.38) (end 107.95 117.475) (width 0.25) (layer B.Cu) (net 5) (status 10))
 (segment (start 107.95 117.475) (end 107.315 116.84) (width 0.25) (layer B.Cu) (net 5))
 (segment (start 107.315 116.84) (end 107.315 104.775) (width 0.25) (layer B.Cu) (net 5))
 (segment (start 107.315 104.775) (end 108.585 103.505) (width 0.25) (layer B.Cu) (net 5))
 (segment (start 108.585 103.505) (end 109.22 102.87) (width 0.25) (layer B.Cu) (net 5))
 (segment (start 109.22 102.87) (end 113.665 102.87) (width 0.25) (layer B.Cu) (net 5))
 (via (at 113.665 102.87) (size 0.8) (drill 0.4) (layers F.Cu B.Cu) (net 5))
 (segment (start 129.23 102.87) (end 129.94 103.58) (width 0.25) (layer F.Cu) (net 5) (status 30))
 (segment (start 113.665 102.87) (end 129.23 102.87) (width 0.25) (layer F.Cu) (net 5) (status 20))
 (segment (start 118.745 97.155) (end 118.745 118.11) (width 0.25) (layer B.Cu) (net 11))
 (segment (start 122.555 93.345) (end 118.745 97.155) (width 0.25) (layer B.Cu) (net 11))
 (segment (start 118.745 118.11) (end 120.015 119.38) (width 0.25) (layer B.Cu) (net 11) (status 20))
 (segment (start 122.555 86.995) (end 122.555 93.345) (width 0.25) (layer B.Cu) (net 11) (status 10))
 (segment (start 122.555 84.455) (end 121.285 84.455) (width 0.25) (layer B.Cu) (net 12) (status 10))
 (segment (start 121.285 84.455) (end 116.205 89.535) (width 0.25) (layer B.Cu) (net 12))
 (segment (start 116.205 115.57) (end 112.395 119.38) (width 0.25) (layer B.Cu) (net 12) (status 20))
 (segment (start 116.205 89.535) (end 116.205 115.57) (width 0.25) (layer B.Cu) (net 12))
 (segment (start 120.65 135.255) (end 120.65 125.095) (width 0.25) (layer F.Cu) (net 15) (status 10))
 (via (at 120.65 125.095) (size 0.8) (drill 0.4) (layers F.Cu B.Cu) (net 15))
 (segment (start 120.65 125.095) (end 116.205 120.65) (width 0.25) (layer B.Cu) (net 15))
 (segment (start 116.205 120.65) (end 116.205 117.475) (width 0.25) (layer B.Cu) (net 15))
 (via (at 116.205 117.475) (size 0.8) (drill 0.4) (layers F.Cu B.Cu) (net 15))
 (segment (start 116.205 117.475) (end 116.205 115.57) (width 0.25) (layer F.Cu) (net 15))
 (segment (start 116.205 115.57) (end 113.665 113.03) (width 0.25) (layer F.Cu) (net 15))
 (segment (start 113.665 113.03) (end 113.665 110.49) (width 0.25) (layer F.Cu) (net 15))
 (segment (start 113.665 110.49) (end 113.665 109.855) (width 0.25) (layer F.Cu) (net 15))
 (via (at 113.665 109.855) (size 0.8) (drill 0.4) (layers F.Cu B.Cu) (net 15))
 (segment (start 113.665 107.315) (end 114.935 106.045) (width 0.25) (layer B.Cu) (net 15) (status 20))
 (segment (start 113.665 109.855) (end 113.665 107.315) (width 0.25) (layer B.Cu) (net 15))
 (segment (start 117.475 119.38) (end 127 128.905) (width 0.25) (layer B.Cu) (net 1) (status 10))
 (segment (start 137.6466 128.905) (end 136.525 128.905) (width 0.25) (layer B.Cu) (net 1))
 (segment (start 149.9362 116.6154) (end 137.6466 128.905) (width 0.25) (layer B.Cu) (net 1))
 (segment (start 127 128.905) (end 136.525 128.905) (width 0.25) (layer B.Cu) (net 1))
 (segment (start 111.125 115.57) (end 114.935 119.38) (width 0.25) (layer F.Cu) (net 13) (status 20))
 (segment (start 111.125 109.855) (end 111.125 115.57) (width 0.25) (layer F.Cu) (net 13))
 (segment (start 109.855 108.585) (end 111.125 109.855) (width 0.25) (layer F.Cu) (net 13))
 (segment (start 109.855 106.045) (end 109.855 108.585) (width 0.25) (layer F.Cu) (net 13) (status 10))
 (segment (start 122.555 117.475) (end 122.555 119.38) (width 0.25) (layer F.Cu) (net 14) (status 20))
 (segment (start 121.285 116.205) (end 122.555 117.475) (width 0.25) (layer F.Cu) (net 14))
 (segment (start 121.285 110.49) (end 121.285 116.205) (width 0.25) (layer F.Cu) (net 14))
 (segment (start 120.65 109.855) (end 121.285 110.49) (width 0.25) (layer F.Cu) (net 14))
 (segment (start 116.205 109.855) (end 120.65 109.855) (width 0.25) (layer F.Cu) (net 14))
 (segment (start 112.395 106.045) (end 116.205 109.855) (width 0.25) (layer F.Cu) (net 14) (status 10))
 (segment (start 108.585 126.365) (end 107.95 126.365) (width 0.25) (layer F.Cu) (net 16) (status 30))
 (segment (start 107.95 126.365) (end 106.68 127.635) (width 0.25) (layer F.Cu) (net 16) (status 10))
 (segment (start 106.68 127.635) (end 106.68 130.81) (width 0.25) (layer F.Cu) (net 16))
 (segment (start 111.125 135.255) (end 113.03 135.255) (width 0.25) (layer F.Cu) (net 16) (status 20))
 (segment (start 106.68 130.81) (end 111.125 135.255) (width 0.25) (layer F.Cu) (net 16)))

